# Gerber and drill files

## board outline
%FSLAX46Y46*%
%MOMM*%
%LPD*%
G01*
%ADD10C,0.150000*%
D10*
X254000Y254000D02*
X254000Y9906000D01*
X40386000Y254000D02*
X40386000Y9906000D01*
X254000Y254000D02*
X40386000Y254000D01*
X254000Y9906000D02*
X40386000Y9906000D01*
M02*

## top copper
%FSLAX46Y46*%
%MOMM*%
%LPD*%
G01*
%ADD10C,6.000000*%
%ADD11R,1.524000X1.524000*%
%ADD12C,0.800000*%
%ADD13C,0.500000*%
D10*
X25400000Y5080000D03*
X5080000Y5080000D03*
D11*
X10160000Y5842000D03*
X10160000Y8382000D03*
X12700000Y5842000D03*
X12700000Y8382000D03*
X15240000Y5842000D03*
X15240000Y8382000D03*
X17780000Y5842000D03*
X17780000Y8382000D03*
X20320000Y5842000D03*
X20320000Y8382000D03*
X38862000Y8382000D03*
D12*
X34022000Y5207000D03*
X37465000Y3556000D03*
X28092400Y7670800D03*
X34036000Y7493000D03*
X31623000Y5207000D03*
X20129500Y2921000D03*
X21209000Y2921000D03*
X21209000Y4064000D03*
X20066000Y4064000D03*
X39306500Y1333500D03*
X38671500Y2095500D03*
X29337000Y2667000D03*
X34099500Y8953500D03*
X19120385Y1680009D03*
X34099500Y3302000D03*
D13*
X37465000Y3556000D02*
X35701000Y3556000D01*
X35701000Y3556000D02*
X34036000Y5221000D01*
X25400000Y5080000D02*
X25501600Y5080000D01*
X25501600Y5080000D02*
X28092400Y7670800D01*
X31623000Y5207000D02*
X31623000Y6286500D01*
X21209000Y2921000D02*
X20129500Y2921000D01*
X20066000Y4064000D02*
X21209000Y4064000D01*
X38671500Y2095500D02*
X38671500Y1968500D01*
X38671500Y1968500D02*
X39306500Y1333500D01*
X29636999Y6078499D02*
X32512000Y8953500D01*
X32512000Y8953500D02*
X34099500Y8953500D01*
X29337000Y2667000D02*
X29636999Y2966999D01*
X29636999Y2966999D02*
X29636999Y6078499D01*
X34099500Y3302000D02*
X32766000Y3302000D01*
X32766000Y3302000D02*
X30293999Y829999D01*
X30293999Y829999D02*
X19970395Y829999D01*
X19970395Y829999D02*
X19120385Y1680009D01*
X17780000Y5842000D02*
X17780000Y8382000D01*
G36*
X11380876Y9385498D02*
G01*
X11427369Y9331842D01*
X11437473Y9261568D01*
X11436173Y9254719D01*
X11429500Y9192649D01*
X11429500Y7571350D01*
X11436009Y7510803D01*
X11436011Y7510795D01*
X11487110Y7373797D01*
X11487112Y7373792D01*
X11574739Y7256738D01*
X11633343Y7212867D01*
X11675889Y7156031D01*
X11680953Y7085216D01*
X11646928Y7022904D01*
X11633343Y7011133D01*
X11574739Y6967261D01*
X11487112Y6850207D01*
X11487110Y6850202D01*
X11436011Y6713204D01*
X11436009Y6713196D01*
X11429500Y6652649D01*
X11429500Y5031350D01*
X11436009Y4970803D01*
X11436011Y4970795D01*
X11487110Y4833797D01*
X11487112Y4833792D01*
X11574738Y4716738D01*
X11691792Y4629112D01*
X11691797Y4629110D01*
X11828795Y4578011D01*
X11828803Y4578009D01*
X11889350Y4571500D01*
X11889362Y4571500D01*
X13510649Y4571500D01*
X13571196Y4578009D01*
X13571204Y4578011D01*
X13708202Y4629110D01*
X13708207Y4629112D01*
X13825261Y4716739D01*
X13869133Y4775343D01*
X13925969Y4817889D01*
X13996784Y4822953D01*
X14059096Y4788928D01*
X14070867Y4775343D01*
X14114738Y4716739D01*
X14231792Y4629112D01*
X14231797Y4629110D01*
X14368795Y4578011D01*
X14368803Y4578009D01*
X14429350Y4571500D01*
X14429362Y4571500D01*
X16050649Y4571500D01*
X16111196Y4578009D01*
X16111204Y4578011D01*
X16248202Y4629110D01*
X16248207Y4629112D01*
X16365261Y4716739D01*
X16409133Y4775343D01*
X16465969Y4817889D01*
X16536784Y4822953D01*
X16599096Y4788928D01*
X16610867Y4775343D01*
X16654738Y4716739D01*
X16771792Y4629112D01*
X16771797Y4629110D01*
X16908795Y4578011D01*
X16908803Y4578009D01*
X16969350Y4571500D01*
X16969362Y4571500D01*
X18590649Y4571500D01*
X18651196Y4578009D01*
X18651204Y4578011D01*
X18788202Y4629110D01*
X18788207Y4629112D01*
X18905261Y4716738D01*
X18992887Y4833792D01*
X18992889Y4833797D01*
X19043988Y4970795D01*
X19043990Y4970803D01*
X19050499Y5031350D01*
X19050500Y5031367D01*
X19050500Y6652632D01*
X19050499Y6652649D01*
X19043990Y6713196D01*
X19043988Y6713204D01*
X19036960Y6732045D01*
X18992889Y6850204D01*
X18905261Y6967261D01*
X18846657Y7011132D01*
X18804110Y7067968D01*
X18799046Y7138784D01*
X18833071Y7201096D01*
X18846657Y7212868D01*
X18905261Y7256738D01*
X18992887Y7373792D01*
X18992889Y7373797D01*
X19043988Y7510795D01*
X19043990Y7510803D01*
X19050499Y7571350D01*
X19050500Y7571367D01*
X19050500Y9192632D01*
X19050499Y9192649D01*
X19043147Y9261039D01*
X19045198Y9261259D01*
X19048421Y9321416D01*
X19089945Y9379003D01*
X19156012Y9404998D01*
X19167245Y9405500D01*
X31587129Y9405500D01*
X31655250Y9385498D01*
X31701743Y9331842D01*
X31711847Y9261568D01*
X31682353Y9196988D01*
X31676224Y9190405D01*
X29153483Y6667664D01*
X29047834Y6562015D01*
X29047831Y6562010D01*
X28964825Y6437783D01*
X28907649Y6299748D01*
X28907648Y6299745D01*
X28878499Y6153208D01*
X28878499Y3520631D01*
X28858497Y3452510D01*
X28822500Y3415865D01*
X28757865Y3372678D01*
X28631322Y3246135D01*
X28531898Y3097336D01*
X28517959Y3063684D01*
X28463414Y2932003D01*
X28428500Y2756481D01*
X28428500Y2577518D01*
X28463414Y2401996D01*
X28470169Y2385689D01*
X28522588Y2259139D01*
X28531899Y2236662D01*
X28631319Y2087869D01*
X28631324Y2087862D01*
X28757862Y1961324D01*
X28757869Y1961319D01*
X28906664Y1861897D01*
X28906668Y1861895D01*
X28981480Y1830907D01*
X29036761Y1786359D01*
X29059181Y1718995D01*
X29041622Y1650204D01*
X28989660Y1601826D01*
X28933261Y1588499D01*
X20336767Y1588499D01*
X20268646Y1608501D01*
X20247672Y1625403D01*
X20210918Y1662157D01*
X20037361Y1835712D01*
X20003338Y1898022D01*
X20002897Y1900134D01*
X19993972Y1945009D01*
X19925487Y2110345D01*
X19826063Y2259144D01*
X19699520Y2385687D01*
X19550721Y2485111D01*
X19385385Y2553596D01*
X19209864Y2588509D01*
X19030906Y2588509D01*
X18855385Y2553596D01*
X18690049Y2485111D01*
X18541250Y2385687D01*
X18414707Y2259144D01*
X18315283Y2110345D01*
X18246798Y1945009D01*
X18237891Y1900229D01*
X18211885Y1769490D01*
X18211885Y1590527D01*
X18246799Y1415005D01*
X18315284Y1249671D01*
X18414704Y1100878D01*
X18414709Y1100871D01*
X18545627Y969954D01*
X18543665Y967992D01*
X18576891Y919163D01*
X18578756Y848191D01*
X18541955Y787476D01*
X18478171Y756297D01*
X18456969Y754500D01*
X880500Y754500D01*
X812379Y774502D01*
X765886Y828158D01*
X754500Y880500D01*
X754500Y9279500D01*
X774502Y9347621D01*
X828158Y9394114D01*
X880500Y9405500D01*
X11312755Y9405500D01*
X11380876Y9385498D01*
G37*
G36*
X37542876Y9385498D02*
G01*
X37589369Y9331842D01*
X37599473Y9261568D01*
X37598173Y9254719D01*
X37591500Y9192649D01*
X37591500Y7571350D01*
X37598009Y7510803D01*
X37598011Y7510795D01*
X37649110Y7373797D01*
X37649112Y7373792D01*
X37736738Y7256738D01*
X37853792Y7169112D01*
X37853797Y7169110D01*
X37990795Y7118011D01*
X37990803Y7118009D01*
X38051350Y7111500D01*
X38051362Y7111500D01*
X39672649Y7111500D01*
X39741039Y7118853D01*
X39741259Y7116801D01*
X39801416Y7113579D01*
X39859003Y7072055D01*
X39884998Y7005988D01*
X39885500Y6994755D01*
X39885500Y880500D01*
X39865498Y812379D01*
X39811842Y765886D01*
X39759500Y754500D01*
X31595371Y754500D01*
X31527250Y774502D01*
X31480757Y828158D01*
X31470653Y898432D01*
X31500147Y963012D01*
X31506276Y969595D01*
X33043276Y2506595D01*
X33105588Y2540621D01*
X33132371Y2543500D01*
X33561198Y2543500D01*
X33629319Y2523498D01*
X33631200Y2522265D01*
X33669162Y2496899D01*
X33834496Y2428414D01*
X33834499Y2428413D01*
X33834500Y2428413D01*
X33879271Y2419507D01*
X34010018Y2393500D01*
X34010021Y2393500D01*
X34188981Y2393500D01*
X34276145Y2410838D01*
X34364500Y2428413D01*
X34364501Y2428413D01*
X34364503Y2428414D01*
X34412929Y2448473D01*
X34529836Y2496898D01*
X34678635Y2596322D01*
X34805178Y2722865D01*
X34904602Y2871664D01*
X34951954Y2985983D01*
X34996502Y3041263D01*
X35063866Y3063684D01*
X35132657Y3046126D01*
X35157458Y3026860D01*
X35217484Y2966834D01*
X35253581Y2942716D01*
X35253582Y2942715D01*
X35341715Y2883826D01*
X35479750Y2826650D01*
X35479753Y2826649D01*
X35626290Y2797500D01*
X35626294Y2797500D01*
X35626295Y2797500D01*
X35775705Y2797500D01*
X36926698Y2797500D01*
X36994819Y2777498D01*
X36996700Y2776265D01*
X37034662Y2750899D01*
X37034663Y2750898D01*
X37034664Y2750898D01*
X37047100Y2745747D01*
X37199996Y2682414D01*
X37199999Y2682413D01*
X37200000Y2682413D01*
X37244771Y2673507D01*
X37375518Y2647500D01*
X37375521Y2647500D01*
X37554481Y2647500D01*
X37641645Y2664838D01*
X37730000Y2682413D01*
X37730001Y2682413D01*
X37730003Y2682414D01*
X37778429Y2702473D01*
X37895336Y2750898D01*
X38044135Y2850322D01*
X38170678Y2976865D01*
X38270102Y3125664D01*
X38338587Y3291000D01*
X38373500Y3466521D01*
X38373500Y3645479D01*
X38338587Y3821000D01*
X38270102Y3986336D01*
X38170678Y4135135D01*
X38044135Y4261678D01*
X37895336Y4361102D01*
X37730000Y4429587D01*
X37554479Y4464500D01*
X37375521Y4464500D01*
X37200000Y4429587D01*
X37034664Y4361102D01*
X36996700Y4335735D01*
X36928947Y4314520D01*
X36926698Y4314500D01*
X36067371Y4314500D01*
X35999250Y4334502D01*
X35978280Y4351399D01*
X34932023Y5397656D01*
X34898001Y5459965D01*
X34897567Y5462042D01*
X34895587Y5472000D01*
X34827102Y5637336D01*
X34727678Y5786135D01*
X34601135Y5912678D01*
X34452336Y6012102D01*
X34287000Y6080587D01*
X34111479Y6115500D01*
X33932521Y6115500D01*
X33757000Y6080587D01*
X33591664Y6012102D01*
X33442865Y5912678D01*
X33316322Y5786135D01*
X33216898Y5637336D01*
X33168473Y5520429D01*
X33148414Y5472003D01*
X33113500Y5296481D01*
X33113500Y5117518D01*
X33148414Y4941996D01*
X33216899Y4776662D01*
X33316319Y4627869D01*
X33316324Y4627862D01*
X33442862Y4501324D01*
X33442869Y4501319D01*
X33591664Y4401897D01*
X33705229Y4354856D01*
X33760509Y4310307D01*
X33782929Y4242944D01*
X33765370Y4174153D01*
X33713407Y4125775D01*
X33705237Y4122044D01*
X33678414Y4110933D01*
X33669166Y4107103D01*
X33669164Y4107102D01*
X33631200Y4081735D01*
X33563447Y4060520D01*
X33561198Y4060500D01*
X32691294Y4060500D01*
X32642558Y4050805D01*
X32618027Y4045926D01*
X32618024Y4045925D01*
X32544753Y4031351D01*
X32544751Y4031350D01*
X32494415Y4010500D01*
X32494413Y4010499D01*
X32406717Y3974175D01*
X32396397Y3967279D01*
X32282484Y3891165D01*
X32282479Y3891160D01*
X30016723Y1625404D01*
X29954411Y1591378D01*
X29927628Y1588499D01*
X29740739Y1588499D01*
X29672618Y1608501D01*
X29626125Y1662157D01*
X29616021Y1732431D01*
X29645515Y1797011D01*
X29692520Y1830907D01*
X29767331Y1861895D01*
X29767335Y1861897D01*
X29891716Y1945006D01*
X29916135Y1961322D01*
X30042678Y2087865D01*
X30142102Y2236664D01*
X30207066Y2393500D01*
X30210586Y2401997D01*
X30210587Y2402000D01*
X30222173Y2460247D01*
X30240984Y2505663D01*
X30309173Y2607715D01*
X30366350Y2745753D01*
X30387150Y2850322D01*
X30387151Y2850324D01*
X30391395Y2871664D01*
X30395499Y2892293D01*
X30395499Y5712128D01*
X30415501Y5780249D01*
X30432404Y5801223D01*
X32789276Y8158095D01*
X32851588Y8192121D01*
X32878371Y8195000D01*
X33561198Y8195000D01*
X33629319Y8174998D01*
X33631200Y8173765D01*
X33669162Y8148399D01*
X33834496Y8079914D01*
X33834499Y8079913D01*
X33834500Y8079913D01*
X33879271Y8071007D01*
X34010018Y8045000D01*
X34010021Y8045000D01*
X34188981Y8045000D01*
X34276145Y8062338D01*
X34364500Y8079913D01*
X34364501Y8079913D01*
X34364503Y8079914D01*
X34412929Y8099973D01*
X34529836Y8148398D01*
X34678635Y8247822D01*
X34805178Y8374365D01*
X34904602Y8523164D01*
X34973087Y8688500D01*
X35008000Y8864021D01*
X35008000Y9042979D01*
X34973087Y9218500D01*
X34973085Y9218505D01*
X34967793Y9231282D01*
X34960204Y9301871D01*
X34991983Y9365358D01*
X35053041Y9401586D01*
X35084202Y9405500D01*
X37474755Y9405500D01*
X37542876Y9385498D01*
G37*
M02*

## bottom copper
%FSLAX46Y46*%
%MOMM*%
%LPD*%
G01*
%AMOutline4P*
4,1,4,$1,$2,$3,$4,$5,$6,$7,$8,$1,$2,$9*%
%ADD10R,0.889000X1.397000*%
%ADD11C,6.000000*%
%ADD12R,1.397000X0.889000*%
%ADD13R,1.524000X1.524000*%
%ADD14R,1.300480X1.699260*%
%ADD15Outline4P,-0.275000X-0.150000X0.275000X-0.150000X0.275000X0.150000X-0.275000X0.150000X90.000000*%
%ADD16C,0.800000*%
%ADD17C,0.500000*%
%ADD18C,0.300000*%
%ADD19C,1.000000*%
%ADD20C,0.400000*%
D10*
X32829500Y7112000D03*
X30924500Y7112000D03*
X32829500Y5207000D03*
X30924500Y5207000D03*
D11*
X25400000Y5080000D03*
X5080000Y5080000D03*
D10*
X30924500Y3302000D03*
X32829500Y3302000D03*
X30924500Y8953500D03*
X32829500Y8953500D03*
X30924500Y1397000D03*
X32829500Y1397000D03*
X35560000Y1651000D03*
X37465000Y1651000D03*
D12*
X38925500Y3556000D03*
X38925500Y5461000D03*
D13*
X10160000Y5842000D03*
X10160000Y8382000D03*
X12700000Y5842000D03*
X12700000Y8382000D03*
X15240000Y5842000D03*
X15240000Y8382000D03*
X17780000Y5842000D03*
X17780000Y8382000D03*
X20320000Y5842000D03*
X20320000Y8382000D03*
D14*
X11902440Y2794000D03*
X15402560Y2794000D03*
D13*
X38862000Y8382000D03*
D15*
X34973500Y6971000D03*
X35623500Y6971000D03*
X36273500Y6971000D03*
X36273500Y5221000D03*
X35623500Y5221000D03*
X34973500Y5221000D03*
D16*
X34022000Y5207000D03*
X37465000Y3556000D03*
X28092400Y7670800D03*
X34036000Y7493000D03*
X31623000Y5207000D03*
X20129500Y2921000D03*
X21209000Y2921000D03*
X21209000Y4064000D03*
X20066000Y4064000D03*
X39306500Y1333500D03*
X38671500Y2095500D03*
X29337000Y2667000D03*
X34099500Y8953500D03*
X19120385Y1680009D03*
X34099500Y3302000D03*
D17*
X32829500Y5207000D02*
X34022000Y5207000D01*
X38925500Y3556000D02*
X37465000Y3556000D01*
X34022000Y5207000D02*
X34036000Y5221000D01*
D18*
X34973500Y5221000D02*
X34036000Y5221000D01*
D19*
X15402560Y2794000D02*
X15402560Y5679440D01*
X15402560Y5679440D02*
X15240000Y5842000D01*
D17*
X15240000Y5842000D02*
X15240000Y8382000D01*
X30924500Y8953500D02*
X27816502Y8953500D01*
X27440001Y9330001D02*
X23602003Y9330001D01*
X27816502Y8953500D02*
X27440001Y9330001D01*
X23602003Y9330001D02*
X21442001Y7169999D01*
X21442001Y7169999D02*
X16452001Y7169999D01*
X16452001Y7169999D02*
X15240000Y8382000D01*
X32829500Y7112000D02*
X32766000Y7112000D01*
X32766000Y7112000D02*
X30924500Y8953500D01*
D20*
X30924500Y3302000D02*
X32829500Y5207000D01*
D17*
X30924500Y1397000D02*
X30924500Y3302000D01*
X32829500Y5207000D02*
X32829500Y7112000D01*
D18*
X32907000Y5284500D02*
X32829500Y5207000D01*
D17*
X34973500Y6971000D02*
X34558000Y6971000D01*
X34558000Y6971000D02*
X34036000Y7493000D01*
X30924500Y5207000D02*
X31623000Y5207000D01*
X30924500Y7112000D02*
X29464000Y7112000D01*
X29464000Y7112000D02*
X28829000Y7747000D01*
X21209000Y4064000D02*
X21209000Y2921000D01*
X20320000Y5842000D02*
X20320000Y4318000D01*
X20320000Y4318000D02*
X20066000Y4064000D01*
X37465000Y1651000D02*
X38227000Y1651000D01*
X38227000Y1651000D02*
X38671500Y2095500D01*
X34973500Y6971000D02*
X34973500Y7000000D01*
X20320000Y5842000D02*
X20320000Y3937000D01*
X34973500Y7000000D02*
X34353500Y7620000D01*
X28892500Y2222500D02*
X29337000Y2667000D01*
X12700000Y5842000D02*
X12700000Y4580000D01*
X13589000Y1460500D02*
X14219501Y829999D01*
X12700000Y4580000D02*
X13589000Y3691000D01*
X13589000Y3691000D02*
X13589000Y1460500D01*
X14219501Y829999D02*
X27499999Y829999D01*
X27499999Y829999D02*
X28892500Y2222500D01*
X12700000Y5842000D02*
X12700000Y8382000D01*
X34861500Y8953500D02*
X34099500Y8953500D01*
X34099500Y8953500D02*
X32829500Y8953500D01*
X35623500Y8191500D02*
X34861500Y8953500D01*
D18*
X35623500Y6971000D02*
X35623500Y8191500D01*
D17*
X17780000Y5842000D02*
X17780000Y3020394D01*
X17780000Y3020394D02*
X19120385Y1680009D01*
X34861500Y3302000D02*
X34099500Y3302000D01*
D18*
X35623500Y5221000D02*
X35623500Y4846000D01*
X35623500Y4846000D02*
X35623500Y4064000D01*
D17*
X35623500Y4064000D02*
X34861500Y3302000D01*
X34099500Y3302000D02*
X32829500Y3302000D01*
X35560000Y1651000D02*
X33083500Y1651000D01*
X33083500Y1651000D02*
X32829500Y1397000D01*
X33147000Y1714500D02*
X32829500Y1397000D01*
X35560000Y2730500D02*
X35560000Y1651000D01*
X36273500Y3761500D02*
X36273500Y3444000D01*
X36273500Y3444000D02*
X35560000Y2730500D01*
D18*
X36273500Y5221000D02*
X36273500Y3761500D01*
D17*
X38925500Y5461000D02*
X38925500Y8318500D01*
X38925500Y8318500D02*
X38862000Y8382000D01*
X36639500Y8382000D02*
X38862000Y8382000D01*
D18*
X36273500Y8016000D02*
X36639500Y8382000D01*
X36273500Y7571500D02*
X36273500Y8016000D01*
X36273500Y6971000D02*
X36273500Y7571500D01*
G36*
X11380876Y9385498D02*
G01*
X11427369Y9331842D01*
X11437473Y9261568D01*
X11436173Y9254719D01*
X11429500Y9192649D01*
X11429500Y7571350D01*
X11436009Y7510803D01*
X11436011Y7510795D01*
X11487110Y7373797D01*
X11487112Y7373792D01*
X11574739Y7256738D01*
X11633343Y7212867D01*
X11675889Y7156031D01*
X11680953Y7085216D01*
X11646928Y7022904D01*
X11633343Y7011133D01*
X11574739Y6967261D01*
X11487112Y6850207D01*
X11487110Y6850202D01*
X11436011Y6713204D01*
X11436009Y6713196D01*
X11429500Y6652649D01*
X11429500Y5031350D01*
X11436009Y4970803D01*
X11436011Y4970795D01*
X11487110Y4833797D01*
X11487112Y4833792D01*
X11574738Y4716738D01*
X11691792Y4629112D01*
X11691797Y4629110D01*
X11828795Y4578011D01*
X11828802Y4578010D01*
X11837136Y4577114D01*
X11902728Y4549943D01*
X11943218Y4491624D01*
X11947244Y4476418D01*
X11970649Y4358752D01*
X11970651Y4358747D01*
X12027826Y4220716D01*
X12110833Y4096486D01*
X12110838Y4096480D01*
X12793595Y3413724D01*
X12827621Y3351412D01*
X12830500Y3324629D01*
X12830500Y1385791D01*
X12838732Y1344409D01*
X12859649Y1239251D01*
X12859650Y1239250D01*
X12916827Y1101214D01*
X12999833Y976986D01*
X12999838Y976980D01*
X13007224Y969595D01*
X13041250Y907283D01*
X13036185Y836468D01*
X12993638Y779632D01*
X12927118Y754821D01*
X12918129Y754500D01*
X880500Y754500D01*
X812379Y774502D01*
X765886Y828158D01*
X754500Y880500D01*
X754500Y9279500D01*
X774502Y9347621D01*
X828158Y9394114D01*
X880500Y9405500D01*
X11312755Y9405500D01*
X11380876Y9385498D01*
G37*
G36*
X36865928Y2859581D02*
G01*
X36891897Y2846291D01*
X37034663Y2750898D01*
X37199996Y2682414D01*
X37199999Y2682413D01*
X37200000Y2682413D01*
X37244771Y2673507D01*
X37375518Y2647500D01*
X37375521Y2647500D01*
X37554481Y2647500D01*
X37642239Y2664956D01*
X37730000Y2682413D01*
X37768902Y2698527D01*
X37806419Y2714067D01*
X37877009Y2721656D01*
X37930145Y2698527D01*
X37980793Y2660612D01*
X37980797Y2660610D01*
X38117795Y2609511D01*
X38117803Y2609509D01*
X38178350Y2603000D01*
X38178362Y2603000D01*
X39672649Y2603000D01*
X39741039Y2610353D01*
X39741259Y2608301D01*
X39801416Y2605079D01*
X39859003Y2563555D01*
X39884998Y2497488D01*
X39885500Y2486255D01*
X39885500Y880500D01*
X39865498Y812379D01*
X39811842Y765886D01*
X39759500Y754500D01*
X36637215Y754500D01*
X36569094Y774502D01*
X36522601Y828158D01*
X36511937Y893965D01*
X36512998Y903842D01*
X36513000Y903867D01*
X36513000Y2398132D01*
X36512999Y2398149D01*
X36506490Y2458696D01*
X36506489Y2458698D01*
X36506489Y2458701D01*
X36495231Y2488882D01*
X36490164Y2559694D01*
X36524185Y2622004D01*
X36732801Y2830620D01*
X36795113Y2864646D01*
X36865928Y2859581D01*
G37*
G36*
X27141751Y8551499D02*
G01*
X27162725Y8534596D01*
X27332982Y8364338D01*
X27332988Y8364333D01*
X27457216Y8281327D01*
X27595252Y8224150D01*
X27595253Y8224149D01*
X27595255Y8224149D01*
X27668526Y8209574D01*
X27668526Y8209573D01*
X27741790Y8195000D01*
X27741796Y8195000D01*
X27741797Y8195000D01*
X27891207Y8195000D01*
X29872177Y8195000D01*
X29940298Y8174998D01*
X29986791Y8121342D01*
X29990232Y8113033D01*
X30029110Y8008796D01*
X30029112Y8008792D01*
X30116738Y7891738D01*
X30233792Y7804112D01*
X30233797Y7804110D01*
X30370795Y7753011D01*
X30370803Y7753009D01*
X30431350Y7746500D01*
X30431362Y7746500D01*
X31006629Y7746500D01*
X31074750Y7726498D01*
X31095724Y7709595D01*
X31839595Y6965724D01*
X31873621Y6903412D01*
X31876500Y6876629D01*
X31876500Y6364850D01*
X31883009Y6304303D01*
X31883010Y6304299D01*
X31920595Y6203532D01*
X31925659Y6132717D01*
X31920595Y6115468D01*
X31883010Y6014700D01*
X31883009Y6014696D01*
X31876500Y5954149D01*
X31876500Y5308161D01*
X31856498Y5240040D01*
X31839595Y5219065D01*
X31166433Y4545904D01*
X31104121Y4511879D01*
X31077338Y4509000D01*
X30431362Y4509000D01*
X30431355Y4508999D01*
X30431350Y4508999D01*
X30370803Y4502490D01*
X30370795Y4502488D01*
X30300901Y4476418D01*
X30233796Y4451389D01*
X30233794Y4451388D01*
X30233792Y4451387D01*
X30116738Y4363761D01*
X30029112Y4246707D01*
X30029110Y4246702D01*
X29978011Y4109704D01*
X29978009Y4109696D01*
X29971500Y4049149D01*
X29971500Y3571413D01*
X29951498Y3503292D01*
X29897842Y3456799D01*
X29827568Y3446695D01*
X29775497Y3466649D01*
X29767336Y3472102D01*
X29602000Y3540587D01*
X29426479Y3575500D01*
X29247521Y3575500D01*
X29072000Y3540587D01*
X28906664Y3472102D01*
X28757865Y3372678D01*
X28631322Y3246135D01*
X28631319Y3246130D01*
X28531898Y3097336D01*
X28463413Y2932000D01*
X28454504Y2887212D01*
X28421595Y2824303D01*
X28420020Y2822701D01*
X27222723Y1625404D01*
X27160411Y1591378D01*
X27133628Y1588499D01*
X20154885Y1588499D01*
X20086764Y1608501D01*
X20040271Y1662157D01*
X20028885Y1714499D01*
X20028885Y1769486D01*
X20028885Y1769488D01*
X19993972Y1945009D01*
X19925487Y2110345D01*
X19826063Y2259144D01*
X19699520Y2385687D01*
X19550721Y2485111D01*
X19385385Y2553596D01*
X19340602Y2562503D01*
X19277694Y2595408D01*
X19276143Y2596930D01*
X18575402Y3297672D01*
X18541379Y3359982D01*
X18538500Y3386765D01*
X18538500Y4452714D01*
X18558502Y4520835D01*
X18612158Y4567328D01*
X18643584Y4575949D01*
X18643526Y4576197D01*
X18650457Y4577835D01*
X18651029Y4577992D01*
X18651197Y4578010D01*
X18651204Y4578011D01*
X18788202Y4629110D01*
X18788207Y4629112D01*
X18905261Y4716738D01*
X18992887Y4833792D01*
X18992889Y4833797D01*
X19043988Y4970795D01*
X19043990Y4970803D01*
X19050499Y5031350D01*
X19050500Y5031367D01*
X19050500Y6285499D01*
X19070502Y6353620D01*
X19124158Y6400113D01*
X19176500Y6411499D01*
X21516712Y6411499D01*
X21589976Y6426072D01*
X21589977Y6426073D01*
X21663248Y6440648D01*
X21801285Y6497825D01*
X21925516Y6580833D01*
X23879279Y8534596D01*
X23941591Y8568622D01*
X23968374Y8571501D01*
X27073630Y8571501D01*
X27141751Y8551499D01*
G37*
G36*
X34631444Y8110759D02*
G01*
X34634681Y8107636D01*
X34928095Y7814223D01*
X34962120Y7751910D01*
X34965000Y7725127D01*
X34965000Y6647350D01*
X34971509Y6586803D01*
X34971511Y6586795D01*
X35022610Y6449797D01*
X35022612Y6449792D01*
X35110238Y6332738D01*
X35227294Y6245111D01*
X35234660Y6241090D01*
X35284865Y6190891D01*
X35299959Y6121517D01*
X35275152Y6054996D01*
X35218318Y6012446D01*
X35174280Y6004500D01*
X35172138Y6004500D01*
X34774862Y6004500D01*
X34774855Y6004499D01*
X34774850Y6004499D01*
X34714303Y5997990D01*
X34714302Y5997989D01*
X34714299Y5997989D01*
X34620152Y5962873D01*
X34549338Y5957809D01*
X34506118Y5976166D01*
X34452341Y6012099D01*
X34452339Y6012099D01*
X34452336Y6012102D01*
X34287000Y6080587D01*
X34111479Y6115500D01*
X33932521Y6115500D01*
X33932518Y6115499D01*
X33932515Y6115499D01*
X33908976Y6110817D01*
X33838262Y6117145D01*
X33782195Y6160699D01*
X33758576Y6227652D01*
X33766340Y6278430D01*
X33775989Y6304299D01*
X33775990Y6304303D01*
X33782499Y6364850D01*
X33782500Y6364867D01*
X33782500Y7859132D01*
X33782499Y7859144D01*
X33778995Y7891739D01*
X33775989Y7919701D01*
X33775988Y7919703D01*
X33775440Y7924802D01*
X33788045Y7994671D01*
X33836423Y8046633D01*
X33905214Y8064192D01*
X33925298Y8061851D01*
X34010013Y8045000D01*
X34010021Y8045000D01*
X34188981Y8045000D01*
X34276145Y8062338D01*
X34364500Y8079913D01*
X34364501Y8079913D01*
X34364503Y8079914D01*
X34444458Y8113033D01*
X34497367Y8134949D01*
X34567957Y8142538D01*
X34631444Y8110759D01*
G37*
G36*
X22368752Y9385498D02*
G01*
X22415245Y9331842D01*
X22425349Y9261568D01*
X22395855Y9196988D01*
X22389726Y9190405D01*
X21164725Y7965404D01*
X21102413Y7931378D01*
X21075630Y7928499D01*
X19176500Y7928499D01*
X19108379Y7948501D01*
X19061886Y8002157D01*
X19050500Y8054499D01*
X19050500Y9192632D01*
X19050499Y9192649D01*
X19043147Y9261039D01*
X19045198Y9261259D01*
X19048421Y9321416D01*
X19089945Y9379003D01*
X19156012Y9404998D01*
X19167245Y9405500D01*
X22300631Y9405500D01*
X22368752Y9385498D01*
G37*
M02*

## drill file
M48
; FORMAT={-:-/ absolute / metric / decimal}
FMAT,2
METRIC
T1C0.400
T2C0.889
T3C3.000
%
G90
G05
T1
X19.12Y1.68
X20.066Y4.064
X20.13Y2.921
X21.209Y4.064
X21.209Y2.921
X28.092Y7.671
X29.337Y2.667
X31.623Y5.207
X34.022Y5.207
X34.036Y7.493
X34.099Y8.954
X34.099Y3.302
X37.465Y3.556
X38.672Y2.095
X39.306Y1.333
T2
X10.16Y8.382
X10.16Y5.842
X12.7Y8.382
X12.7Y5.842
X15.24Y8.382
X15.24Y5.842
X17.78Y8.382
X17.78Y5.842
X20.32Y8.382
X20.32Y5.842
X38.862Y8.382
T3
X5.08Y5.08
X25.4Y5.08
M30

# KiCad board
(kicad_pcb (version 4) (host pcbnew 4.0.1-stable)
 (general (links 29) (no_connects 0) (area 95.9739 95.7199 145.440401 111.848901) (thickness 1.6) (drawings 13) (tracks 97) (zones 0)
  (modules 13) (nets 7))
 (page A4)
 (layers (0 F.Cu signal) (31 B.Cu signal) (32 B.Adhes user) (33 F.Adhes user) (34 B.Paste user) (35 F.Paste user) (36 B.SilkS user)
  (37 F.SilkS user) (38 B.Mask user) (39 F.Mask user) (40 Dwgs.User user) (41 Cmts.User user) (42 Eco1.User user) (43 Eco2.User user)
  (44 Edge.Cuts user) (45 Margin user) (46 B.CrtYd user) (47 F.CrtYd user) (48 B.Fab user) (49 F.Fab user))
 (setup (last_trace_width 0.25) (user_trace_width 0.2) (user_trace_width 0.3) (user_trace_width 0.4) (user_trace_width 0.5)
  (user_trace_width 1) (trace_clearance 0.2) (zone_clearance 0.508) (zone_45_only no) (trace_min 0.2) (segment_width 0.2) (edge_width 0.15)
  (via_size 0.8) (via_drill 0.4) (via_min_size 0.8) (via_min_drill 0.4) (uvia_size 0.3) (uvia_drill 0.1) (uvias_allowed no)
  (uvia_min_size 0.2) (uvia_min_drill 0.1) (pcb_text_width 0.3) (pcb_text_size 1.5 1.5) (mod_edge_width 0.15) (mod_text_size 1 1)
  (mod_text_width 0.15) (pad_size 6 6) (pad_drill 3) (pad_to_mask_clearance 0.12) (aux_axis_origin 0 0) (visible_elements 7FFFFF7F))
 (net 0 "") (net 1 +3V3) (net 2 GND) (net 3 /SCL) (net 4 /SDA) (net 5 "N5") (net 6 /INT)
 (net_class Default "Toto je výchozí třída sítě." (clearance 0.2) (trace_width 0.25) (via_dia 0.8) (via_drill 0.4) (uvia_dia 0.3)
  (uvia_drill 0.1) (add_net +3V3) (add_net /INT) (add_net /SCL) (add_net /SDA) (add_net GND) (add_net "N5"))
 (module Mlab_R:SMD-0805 (layer B.Cu) (at 31.877 -7.112 180)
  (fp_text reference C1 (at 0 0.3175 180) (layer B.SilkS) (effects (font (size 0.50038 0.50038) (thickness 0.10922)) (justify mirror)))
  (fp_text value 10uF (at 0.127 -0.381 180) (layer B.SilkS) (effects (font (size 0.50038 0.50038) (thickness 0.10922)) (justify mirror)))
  (pad 1 smd rect (at -0.9525 0 180) (size 0.889 1.397) (layers B.Cu B.Paste B.Mask) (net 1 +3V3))
  (pad 2 smd rect (at 0.9525 0 180) (size 0.889 1.397) (layers B.Cu B.Paste B.Mask) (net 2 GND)))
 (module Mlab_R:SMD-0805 (layer B.Cu) (at 31.877 -5.207 180)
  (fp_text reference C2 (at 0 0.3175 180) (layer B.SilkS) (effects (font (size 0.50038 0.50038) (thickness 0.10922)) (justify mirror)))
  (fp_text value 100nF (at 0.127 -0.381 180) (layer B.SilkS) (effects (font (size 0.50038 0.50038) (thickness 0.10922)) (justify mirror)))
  (pad 1 smd rect (at -0.9525 0 180) (size 0.889 1.397) (layers B.Cu B.Paste B.Mask) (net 1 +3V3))
  (pad 2 smd rect (at 0.9525 0 180) (size 0.889 1.397) (layers B.Cu B.Paste B.Mask) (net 2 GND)))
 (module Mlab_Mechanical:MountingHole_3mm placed (layer F.Cu) (at 25.4 -5.08)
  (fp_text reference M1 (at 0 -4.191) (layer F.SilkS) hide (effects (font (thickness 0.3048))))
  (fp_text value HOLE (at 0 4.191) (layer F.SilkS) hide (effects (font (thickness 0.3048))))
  (pad 1 thru_hole circle (at 0 0) (size 6 6) (drill 3) (layers *.Cu *.Adhes *.Mask) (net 2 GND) (clearance 1) (zone_connect 2)))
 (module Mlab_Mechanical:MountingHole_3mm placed (layer F.Cu) (at 5.08 -5.08)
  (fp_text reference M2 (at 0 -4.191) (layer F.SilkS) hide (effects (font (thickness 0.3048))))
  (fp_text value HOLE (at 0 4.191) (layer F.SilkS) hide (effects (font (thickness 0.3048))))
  (pad 1 thru_hole circle (at 0 0) (size 6 6) (drill 3) (layers *.Cu *.Adhes *.Mask) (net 2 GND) (clearance 1) (zone_connect 2)))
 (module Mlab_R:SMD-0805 (layer B.Cu) (at 31.877 -3.302)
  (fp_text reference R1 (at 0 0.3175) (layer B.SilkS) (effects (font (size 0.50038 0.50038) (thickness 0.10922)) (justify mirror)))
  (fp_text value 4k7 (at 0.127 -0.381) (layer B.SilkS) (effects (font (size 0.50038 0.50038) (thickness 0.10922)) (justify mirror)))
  (pad 1 smd rect (at -0.9525 0) (size 0.889 1.397) (layers B.Cu B.Paste B.Mask) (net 1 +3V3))
  (pad 2 smd rect (at 0.9525 0) (size 0.889 1.397) (layers B.Cu B.Paste B.Mask) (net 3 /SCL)))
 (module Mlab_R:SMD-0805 (layer B.Cu) (at 31.877 -8.9535)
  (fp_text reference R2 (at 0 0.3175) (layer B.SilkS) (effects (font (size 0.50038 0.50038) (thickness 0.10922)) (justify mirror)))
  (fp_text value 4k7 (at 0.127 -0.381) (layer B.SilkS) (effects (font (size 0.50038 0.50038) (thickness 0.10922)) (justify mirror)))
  (pad 1 smd rect (at -0.9525 0) (size 0.889 1.397) (layers B.Cu B.Paste B.Mask) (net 1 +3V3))
  (pad 2 smd rect (at 0.9525 0) (size 0.889 1.397) (layers B.Cu B.Paste B.Mask) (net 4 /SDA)))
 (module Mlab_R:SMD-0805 (layer B.Cu) (at 31.877 -1.397)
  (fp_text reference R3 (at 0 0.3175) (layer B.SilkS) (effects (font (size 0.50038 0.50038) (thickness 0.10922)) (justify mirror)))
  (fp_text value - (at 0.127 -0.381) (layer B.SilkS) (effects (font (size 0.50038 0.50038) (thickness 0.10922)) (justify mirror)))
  (pad 1 smd rect (at -0.9525 0) (size 0.889 1.397) (layers B.Cu B.Paste B.Mask) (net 1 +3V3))
  (pad 2 smd rect (at 0.9525 0) (size 0.889 1.397) (layers B.Cu B.Paste B.Mask) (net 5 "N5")))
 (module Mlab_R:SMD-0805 (layer B.Cu) (at 36.5125 -1.651)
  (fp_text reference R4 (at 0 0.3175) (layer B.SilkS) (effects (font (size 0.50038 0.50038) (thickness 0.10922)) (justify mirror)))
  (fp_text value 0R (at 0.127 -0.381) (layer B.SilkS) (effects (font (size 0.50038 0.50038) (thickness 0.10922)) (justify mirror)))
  (pad 1 smd rect (at -0.9525 0) (size 0.889 1.397) (layers B.Cu B.Paste B.Mask) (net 5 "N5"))
  (pad 2 smd rect (at 0.9525 0) (size 0.889 1.397) (layers B.Cu B.Paste B.Mask) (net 2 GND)))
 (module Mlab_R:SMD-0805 (layer B.Cu) (at 38.9255 -4.5085 90)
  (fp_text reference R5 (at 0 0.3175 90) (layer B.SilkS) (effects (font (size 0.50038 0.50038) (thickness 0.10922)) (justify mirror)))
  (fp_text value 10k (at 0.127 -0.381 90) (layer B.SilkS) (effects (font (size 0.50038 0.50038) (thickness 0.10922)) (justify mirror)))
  (pad 1 smd rect (at -0.9525 0 90) (size 0.889 1.397) (layers B.Cu B.Paste B.Mask) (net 1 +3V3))
  (pad 2 smd rect (at 0.9525 0 90) (size 0.889 1.397) (layers B.Cu B.Paste B.Mask) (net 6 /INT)))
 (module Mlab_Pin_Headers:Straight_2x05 (layer F.Cu) (at 15.24 -7.112 90)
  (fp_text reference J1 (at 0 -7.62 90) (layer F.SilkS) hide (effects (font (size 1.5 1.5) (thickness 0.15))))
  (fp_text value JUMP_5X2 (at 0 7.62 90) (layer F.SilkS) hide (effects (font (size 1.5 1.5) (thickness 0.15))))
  (pad 1 thru_hole rect (at -1.27 -5.08 90) (size 1.524 1.524) (drill 0.889) (layers *.Cu *.Mask F.SilkS) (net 2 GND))
  (pad 2 thru_hole rect (at 1.27 -5.08 90) (size 1.524 1.524) (drill 0.889) (layers *.Cu *.Mask F.SilkS) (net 2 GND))
  (pad 3 thru_hole rect (at -1.27 -2.54 90) (size 1.524 1.524) (drill 0.889) (layers *.Cu *.Mask F.SilkS) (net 4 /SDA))
  (pad 4 thru_hole rect (at 1.27 -2.54 90) (size 1.524 1.524) (drill 0.889) (layers *.Cu *.Mask F.SilkS) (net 4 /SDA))
  (pad 5 thru_hole rect (at -1.27 0 90) (size 1.524 1.524) (drill 0.889) (layers *.Cu *.Mask F.SilkS) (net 1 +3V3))
  (pad 6 thru_hole rect (at 1.27 0 90) (size 1.524 1.524) (drill 0.889) (layers *.Cu *.Mask F.SilkS) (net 1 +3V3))
  (pad 7 thru_hole rect (at -1.27 2.54 90) (size 1.524 1.524) (drill 0.889) (layers *.Cu *.Mask F.SilkS) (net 3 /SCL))
  (pad 8 thru_hole rect (at 1.27 2.54 90) (size 1.524 1.524) (drill 0.889) (layers *.Cu *.Mask F.SilkS) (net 3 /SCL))
  (pad 9 thru_hole rect (at -1.27 5.08 90) (size 1.524 1.524) (drill 0.889) (layers *.Cu *.Mask F.SilkS) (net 2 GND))
  (pad 10 thru_hole rect (at 1.27 5.08 90) (size 1.524 1.524) (drill 0.889) (layers *.Cu *.Mask F.SilkS) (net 2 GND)))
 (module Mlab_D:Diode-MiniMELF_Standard (layer B.Cu) (at 13.6525 -2.794)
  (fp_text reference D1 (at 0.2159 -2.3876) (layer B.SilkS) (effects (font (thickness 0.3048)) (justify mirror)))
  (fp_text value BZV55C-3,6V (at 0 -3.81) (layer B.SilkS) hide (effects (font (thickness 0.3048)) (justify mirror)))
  (pad 1 smd rect (at -1.75006 0) (size 1.30048 1.69926) (layers B.Cu B.Paste B.Mask) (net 2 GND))
  (pad 2 smd rect (at 1.75006 0) (size 1.30048 1.69926) (layers B.Cu B.Paste B.Mask) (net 1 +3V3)))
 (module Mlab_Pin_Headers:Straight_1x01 (layer F.Cu) (at 38.862 -8.382)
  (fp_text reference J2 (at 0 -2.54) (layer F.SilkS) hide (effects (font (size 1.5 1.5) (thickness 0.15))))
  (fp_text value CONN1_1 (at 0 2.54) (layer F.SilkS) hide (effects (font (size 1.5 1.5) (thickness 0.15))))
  (pad 1 thru_hole rect (at 0 0) (size 1.524 1.524) (drill 0.889) (layers *.Cu *.Mask F.SilkS) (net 6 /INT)))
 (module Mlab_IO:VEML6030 (layer B.Cu) (at 35.6235 -6.096 90)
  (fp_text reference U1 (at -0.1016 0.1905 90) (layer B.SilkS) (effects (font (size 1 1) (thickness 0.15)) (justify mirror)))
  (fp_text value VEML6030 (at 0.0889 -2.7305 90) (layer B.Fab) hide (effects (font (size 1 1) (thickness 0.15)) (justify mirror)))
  (pad 1 smd trapezoid (at 0.875 -0.65 90) (size 0.55 0.3) (layers B.Cu B.Paste B.Mask) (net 2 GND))
  (pad 2 smd trapezoid (at 0.875 0 90) (size 0.55 0.3) (layers B.Cu B.Paste B.Mask) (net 4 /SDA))
  (pad 3 smd trapezoid (at 0.875 0.65 90) (size 0.55 0.3) (layers B.Cu B.Paste B.Mask) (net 6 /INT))
  (pad 4 smd trapezoid (at -0.875 0.65 90) (size 0.55 0.3) (layers B.Cu B.Paste B.Mask) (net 5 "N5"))
  (pad 5 smd trapezoid (at -0.875 0 90) (size 0.55 0.3) (layers B.Cu B.Paste B.Mask) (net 3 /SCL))
  (pad 6 smd trapezoid (at -0.875 -0.65 90) (size 0.55 0.3) (layers B.Cu B.Paste B.Mask) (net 1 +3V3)))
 (gr_line (start 0.254 -0.254) (end 0.254 -9.906) (angle 90) (layer Edge.Cuts) (width 0.15))
 (gr_line (start 40.386 -0.254) (end 40.386 -9.906) (angle 90) (layer Edge.Cuts) (width 0.15))
 (gr_line (start 0.254 -0.254) (end 40.386 -0.254) (angle 90) (layer Edge.Cuts) (width 0.15))
 (gr_line (start 0.254 -9.906) (end 40.386 -9.906) (angle 90) (layer Edge.Cuts) (width 0.15))
 (segment (start 32.8295 -5.207) (end 34.022 -5.207) (width 0.5) (layer B.Cu) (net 1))
 (via (at 34.022 -5.207) (size 0.8) (drill 0.4) (layers F.Cu B.Cu) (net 1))
 (segment (start 38.9255 -3.556) (end 37.465 -3.556) (width 0.5) (layer B.Cu) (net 1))
 (via (at 37.465 -3.556) (size 0.8) (drill 0.4) (layers F.Cu B.Cu) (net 1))
 (segment (start 34.022 -5.207) (end 34.036 -5.221) (width 0.5) (layer B.Cu) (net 1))
 (segment (start 34.9735 -5.221) (end 34.036 -5.221) (width 0.3) (layer B.Cu) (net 1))
 (segment (start 37.465 -3.556) (end 35.701 -3.556) (width 0.5) (layer F.Cu) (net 1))
 (segment (start 35.701 -3.556) (end 34.036 -5.221) (width 0.5) (layer F.Cu) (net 1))
 (segment (start 15.40256 -2.794) (end 15.40256 -5.67944) (width 1) (layer B.Cu) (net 1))
 (segment (start 15.40256 -5.67944) (end 15.24 -5.842) (width 1) (layer B.Cu) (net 1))
 (segment (start 15.24 -5.842) (end 15.24 -8.382) (width 0.5) (layer B.Cu) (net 1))
 (segment (start 30.9245 -8.9535) (end 27.816502 -8.9535) (width 0.5) (layer B.Cu) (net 1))
 (segment (start 27.440001 -9.330001) (end 23.602003 -9.330001) (width 0.5) (layer B.Cu) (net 1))
 (segment (start 27.816502 -8.9535) (end 27.440001 -9.330001) (width 0.5) (layer B.Cu) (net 1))
 (segment (start 23.602003 -9.330001) (end 21.442001 -7.169999) (width 0.5) (layer B.Cu) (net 1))
 (segment (start 21.442001 -7.169999) (end 16.452001 -7.169999) (width 0.5) (layer B.Cu) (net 1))
 (segment (start 16.452001 -7.169999) (end 15.24 -8.382) (width 0.5) (layer B.Cu) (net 1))
 (segment (start 32.8295 -7.112) (end 32.766 -7.112) (width 0.5) (layer B.Cu) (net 1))
 (segment (start 32.766 -7.112) (end 30.9245 -8.9535) (width 0.5) (layer B.Cu) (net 1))
 (segment (start 30.9245 -3.302) (end 32.8295 -5.207) (width 0.4) (layer B.Cu) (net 1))
 (segment (start 30.9245 -1.397) (end 30.9245 -3.302) (width 0.5) (layer B.Cu) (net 1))
 (segment (start 32.8295 -5.207) (end 32.8295 -7.112) (width 0.5) (layer B.Cu) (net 1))
 (segment (start 32.907 -5.2845) (end 32.8295 -5.207) (width 0.3) (layer B.Cu) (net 1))
 (segment (start 25.4 -5.08) (end 25.5016 -5.08) (width 0.5) (layer F.Cu) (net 2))
 (segment (start 25.5016 -5.08) (end 28.0924 -7.6708) (width 0.5) (layer F.Cu) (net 2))
 (via (at 28.0924 -7.6708) (size 0.8) (drill 0.4) (layers F.Cu B.Cu) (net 2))
 (segment (start 34.9735 -6.971) (end 34.558 -6.971) (width 0.5) (layer B.Cu) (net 2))
 (segment (start 34.558 -6.971) (end 34.036 -7.493) (width 0.5) (layer B.Cu) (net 2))
 (via (at 34.036 -7.493) (size 0.8) (drill 0.4) (layers F.Cu B.Cu) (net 2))
 (segment (start 31.623 -5.207) (end 31.623 -6.2865) (width 0.5) (layer F.Cu) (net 2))
 (segment (start 30.9245 -5.207) (end 31.623 -5.207) (width 0.5) (layer B.Cu) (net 2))
 (via (at 31.623 -5.207) (size 0.8) (drill 0.4) (layers F.Cu B.Cu) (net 2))
 (segment (start 30.9245 -7.112) (end 29.464 -7.112) (width 0.5) (layer B.Cu) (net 2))
 (segment (start 29.464 -7.112) (end 28.829 -7.747) (width 0.5) (layer B.Cu) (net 2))
 (segment (start 21.209 -2.921) (end 20.1295 -2.921) (width 0.5) (layer F.Cu) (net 2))
 (via (at 20.1295 -2.921) (size 0.8) (drill 0.4) (layers F.Cu B.Cu) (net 2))
 (segment (start 21.209 -4.064) (end 21.209 -2.921) (width 0.5) (layer B.Cu) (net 2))
 (via (at 21.209 -2.921) (size 0.8) (drill 0.4) (layers F.Cu B.Cu) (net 2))
 (segment (start 20.066 -4.064) (end 21.209 -4.064) (width 0.5) (layer F.Cu) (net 2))
 (via (at 21.209 -4.064) (size 0.8) (drill 0.4) (layers F.Cu B.Cu) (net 2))
 (segment (start 20.32 -5.842) (end 20.32 -4.318) (width 0.5) (layer B.Cu) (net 2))
 (segment (start 20.32 -4.318) (end 20.066 -4.064) (width 0.5) (layer B.Cu) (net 2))
 (via (at 20.066 -4.064) (size 0.8) (drill 0.4) (layers F.Cu B.Cu) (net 2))
 (segment (start 38.6715 -2.0955) (end 38.6715 -1.9685) (width 0.5) (layer F.Cu) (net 2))
 (segment (start 38.6715 -1.9685) (end 39.3065 -1.3335) (width 0.5) (layer F.Cu) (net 2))
 (via (at 39.3065 -1.3335) (size 0.8) (drill 0.4) (layers F.Cu B.Cu) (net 2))
 (segment (start 37.465 -1.651) (end 38.227 -1.651) (width 0.5) (layer B.Cu) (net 2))
 (segment (start 38.227 -1.651) (end 38.6715 -2.0955) (width 0.5) (layer B.Cu) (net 2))
 (via (at 38.6715 -2.0955) (size 0.8) (drill 0.4) (layers F.Cu B.Cu) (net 2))
 (segment (start 34.9735 -6.971) (end 34.9735 -7) (width 0.5) (layer B.Cu) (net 2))
 (segment (start 20.32 -5.842) (end 20.32 -3.937) (width 0.5) (layer B.Cu) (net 2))
 (segment (start 34.9735 -7) (end 34.3535 -7.62) (width 0.5) (layer B.Cu) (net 2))
 (segment (start 28.8925 -2.2225) (end 29.337 -2.667) (width 0.5) (layer B.Cu) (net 4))
 (via (at 29.337 -2.667) (size 0.8) (drill 0.4) (layers F.Cu B.Cu) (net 4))
 (segment (start 12.7 -5.842) (end 12.7 -4.58) (width 0.5) (layer B.Cu) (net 4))
 (segment (start 13.589 -1.4605) (end 14.219501 -0.829999) (width 0.5) (layer B.Cu) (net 4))
 (segment (start 12.7 -4.58) (end 13.589 -3.691) (width 0.5) (layer B.Cu) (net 4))
 (segment (start 13.589 -3.691) (end 13.589 -1.4605) (width 0.5) (layer B.Cu) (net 4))
 (segment (start 14.219501 -0.829999) (end 27.499999 -0.829999) (width 0.5) (layer B.Cu) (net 4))
 (segment (start 27.499999 -0.829999) (end 28.8925 -2.2225) (width 0.5) (layer B.Cu) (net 4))
 (via (at 34.0995 -8.9535) (size 0.8) (drill 0.4) (layers F.Cu B.Cu) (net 4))
 (segment (start 12.7 -5.842) (end 12.7 -8.382) (width 0.5) (layer B.Cu) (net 4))
 (segment (start 34.8615 -8.9535) (end 34.0995 -8.9535) (width 0.5) (layer B.Cu) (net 4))
 (segment (start 34.0995 -8.9535) (end 32.8295 -8.9535) (width 0.5) (layer B.Cu) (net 4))
 (segment (start 29.636999 -6.078499) (end 32.512 -8.9535) (width 0.5) (layer F.Cu) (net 4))
 (segment (start 32.512 -8.9535) (end 34.0995 -8.9535) (width 0.5) (layer F.Cu) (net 4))
 (segment (start 29.337 -2.667) (end 29.636999 -2.966999) (width 0.5) (layer F.Cu) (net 4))
 (segment (start 29.636999 -2.966999) (end 29.636999 -6.078499) (width 0.5) (layer F.Cu) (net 4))
 (segment (start 35.6235 -8.1915) (end 34.8615 -8.9535) (width 0.5) (layer B.Cu) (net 4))
 (segment (start 35.6235 -6.971) (end 35.6235 -8.1915) (width 0.3) (layer B.Cu) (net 4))
 (segment (start 34.0995 -3.302) (end 32.766 -3.302) (width 0.5) (layer F.Cu) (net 3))
 (segment (start 32.766 -3.302) (end 30.293999 -0.829999) (width 0.5) (layer F.Cu) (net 3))
 (segment (start 30.293999 -0.829999) (end 19.970395 -0.829999) (width 0.5) (layer F.Cu) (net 3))
 (segment (start 19.970395 -0.829999) (end 19.120385 -1.680009) (width 0.5) (layer F.Cu) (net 3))
 (segment (start 17.78 -5.842) (end 17.78 -3.020394) (width 0.5) (layer B.Cu) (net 3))
 (segment (start 17.78 -3.020394) (end 19.120385 -1.680009) (width 0.5) (layer B.Cu) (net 3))
 (via (at 19.120385 -1.680009) (size 0.8) (drill 0.4) (layers F.Cu B.Cu) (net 3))
 (via (at 34.0995 -3.302) (size 0.8) (drill 0.4) (layers F.Cu B.Cu) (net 3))
 (segment (start 34.8615 -3.302) (end 34.0995 -3.302) (width 0.5) (layer B.Cu) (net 3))
 (segment (start 35.6235 -5.221) (end 35.6235 -4.846) (width 0.3) (layer B.Cu) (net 3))
 (segment (start 35.6235 -4.846) (end 35.6235 -4.064) (width 0.3) (layer B.Cu) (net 3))
 (segment (start 35.6235 -4.064) (end 34.8615 -3.302) (width 0.5) (layer B.Cu) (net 3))
 (segment (start 17.78 -5.842) (end 17.78 -8.382) (width 0.5) (layer F.Cu) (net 3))
 (segment (start 34.0995 -3.302) (end 32.8295 -3.302) (width 0.5) (layer B.Cu) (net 3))
 (segment (start 35.56 -1.651) (end 33.0835 -1.651) (width 0.5) (layer B.Cu) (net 5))
 (segment (start 33.0835 -1.651) (end 32.8295 -1.397) (width 0.5) (layer B.Cu) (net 5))
 (segment (start 33.147 -1.7145) (end 32.8295 -1.397) (width 0.5) (layer B.Cu) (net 5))
 (segment (start 35.56 -2.7305) (end 35.56 -1.651) (width 0.5) (layer B.Cu) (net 5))
 (segment (start 36.2735 -3.7615) (end 36.2735 -3.444) (width 0.5) (layer B.Cu) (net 5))
 (segment (start 36.2735 -3.444) (end 35.56 -2.7305) (width 0.5) (layer B.Cu) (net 5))
 (segment (start 36.2735 -5.221) (end 36.2735 -3.7615) (width 0.3) (layer B.Cu) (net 5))
 (segment (start 38.9255 -5.461) (end 38.9255 -8.3185) (width 0.5) (layer B.Cu) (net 6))
 (segment (start 38.9255 -8.3185) (end 38.862 -8.382) (width 0.5) (layer B.Cu) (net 6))
 (segment (start 36.6395 -8.382) (end 38.862 -8.382) (width 0.5) (layer B.Cu) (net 6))
 (segment (start 36.2735 -8.016) (end 36.6395 -8.382) (width 0.3) (layer B.Cu) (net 6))
 (segment (start 36.2735 -7.5715) (end 36.2735 -8.016) (width 0.3) (layer B.Cu) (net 6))
 (segment (start 36.2735 -6.971) (end 36.2735 -7.5715) (width 0.3) (layer B.Cu) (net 6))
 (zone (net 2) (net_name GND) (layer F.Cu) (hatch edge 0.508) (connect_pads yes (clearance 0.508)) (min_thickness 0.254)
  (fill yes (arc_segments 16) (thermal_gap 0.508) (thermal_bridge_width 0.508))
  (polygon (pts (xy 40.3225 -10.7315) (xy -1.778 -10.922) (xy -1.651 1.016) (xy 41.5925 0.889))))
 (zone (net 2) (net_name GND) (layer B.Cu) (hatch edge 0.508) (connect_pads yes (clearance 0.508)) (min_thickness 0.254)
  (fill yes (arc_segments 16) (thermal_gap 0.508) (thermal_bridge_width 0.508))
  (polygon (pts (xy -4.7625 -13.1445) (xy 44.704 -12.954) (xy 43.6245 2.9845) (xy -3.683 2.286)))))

